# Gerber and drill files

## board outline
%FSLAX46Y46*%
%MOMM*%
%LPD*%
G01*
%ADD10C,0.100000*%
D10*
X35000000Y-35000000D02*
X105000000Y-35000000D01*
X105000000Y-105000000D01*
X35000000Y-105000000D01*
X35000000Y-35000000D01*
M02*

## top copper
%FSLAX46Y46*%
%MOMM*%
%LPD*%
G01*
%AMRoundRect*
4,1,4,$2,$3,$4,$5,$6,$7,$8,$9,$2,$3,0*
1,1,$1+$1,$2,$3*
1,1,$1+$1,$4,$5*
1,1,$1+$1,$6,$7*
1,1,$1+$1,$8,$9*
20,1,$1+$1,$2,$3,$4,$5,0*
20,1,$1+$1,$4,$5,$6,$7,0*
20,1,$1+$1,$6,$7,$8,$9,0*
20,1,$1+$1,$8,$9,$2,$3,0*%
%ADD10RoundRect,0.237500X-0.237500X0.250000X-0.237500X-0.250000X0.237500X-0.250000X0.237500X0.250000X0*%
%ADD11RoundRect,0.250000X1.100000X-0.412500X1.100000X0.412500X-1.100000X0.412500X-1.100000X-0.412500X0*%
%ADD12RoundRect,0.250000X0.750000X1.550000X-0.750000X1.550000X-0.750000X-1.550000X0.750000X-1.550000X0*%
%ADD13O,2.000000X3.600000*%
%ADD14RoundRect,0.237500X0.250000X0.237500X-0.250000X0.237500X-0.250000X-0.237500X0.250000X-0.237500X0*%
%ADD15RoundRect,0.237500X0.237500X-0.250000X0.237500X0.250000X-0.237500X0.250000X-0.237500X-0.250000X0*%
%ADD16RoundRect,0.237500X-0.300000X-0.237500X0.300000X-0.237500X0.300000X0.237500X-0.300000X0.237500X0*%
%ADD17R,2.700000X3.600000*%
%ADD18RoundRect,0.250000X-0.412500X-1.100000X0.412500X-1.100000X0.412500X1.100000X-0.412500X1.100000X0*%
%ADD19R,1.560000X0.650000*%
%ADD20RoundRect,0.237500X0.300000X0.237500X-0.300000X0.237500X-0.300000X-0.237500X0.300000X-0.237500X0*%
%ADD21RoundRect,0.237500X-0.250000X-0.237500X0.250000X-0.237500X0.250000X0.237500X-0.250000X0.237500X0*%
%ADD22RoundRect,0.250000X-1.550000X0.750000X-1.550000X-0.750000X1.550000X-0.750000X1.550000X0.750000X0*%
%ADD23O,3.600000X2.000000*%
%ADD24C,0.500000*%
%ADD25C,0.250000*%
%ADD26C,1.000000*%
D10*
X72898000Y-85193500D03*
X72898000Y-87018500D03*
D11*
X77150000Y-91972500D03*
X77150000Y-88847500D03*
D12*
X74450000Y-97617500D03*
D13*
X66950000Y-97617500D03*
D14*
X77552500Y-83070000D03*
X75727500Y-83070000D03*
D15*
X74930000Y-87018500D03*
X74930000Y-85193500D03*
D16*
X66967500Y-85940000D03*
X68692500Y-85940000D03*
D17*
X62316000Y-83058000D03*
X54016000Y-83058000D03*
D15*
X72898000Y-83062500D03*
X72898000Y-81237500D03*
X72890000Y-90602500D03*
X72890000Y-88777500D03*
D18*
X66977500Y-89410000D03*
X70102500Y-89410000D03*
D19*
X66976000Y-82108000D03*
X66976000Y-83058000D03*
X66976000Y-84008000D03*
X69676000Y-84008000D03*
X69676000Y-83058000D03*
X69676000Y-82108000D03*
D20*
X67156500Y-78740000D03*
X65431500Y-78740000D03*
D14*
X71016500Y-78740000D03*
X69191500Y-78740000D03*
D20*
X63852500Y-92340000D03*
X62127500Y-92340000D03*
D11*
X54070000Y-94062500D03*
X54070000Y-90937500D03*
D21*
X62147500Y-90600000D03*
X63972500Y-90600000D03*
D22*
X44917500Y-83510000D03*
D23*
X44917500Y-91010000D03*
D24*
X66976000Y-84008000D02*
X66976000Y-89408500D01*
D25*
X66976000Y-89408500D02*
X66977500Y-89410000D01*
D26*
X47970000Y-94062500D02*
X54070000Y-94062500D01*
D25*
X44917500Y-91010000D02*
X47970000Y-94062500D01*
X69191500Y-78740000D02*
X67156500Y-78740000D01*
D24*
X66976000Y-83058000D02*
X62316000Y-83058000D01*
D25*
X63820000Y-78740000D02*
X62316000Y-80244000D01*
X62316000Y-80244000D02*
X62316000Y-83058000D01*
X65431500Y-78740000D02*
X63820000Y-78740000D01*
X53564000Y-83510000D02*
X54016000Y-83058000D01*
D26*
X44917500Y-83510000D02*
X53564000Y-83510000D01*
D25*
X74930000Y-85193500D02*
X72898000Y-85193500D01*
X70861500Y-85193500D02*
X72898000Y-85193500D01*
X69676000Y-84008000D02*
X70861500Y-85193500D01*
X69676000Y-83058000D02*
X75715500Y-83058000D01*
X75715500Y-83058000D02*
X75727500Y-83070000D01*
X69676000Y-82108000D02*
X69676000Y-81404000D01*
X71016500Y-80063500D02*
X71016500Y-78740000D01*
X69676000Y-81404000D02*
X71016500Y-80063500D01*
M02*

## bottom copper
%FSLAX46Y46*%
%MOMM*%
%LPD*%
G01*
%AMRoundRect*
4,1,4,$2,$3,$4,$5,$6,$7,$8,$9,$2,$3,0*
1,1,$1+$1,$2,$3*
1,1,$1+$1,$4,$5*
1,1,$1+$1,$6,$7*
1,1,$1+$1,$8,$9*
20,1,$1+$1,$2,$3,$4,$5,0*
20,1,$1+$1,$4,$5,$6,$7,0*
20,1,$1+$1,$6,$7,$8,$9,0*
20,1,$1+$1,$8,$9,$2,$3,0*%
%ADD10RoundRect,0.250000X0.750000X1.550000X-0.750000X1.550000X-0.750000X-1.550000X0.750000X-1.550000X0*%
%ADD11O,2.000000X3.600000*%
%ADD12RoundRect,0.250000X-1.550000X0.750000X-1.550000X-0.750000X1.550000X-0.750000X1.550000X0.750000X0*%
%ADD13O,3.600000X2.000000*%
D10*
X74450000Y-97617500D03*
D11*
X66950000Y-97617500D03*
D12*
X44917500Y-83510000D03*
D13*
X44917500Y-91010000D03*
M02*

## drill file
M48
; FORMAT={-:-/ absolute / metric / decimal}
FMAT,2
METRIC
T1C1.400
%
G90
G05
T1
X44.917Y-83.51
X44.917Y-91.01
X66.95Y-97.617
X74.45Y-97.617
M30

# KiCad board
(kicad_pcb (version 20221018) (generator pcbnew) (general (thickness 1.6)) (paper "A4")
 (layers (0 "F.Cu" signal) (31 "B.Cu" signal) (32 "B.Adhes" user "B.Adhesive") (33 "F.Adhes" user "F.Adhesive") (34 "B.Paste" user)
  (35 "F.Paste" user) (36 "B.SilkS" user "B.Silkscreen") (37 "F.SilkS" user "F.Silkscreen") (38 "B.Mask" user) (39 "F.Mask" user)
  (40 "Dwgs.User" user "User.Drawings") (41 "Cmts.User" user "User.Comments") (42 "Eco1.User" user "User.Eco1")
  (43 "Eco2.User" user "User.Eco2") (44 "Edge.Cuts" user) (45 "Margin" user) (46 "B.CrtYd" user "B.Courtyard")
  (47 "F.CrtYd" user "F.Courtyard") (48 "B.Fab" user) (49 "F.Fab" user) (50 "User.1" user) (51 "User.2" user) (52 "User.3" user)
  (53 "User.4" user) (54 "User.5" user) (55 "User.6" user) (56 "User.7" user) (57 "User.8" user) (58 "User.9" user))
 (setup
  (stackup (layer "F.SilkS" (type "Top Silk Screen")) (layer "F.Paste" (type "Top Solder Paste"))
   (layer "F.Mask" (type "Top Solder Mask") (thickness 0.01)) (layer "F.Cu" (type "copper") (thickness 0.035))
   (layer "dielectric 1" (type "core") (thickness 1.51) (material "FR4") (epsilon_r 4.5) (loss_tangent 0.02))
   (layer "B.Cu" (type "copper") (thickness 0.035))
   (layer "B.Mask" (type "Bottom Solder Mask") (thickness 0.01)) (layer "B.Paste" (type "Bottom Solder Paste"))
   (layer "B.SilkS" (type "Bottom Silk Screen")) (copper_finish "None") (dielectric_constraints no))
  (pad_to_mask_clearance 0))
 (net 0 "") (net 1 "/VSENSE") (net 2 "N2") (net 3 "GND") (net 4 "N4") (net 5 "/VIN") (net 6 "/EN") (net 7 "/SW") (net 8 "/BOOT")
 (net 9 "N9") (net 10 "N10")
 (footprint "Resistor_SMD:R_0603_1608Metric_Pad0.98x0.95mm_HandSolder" (layer "F.Cu") (at 72.898 86.106 -90)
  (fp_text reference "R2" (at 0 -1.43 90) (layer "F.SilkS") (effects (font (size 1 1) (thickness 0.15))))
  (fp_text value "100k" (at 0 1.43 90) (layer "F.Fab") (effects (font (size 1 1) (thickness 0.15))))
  (pad "1" smd roundrect (at -0.9125 0 270) (size 0.975 0.95) (layers "F.Cu" "F.Paste" "F.Mask") (roundrect_rratio 0.25) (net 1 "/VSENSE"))
  (pad "2" smd roundrect (at 0.9125 0 270) (size 0.975 0.95) (layers "F.Cu" "F.Paste" "F.Mask") (roundrect_rratio 0.25) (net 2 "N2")))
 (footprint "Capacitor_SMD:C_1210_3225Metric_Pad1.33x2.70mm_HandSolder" (layer "F.Cu") (at 77.15 90.41 90)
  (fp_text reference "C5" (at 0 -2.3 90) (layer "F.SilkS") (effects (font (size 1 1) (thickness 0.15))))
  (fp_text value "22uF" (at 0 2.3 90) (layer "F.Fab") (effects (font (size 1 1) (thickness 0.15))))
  (pad "1" smd roundrect (at -1.5625 0 90) (size 1.325 2.7) (layers "F.Cu" "F.Paste" "F.Mask") (roundrect_rratio 0.188679) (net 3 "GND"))
  (pad "2" smd roundrect (at 1.5625 0 90) (size 1.325 2.7) (layers "F.Cu" "F.Paste" "F.Mask") (roundrect_rratio 0.188679) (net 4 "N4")))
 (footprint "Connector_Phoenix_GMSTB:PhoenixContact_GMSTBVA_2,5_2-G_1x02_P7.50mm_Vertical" (layer "F.Cu") (at 70.76 97.6175 180)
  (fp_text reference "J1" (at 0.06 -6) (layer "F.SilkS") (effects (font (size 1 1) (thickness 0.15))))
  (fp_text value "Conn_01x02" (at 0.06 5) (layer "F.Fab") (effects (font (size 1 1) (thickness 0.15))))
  (pad "1" thru_hole roundrect (at -3.69 0 180) (size 2 3.6) (drill 1.4) (layers "*.Cu" "*.Mask") (roundrect_rratio 0.125) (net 3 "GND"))
  (pad "2" thru_hole oval (at 3.81 0 180) (size 2 3.6) (drill 1.4) (layers "*.Cu" "*.Mask") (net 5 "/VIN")))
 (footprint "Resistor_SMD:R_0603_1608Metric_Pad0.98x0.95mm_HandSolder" (layer "F.Cu") (at 76.64 83.07 180)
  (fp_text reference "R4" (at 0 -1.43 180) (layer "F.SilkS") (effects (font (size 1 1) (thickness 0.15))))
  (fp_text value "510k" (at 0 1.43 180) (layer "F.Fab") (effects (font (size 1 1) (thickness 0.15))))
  (pad "1" smd roundrect (at -0.9125 0 180) (size 0.975 0.95) (layers "F.Cu" "F.Paste" "F.Mask") (roundrect_rratio 0.25) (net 5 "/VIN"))
  (pad "2" smd roundrect (at 0.9125 0 180) (size 0.975 0.95) (layers "F.Cu" "F.Paste" "F.Mask") (roundrect_rratio 0.25) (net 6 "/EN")))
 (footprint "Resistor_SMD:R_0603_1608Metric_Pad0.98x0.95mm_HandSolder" (layer "F.Cu") (at 74.93 86.106 90)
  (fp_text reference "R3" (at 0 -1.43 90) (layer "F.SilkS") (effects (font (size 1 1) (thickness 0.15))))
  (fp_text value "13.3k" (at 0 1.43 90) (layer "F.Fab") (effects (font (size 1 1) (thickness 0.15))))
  (pad "1" smd roundrect (at -0.9125 0 90) (size 0.975 0.95) (layers "F.Cu" "F.Paste" "F.Mask") (roundrect_rratio 0.25) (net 3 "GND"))
  (pad "2" smd roundrect (at 0.9125 0 90) (size 0.975 0.95) (layers "F.Cu" "F.Paste" "F.Mask") (roundrect_rratio 0.25) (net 1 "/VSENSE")))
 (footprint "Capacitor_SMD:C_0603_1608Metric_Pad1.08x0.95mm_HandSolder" (layer "F.Cu") (at 67.83 85.94)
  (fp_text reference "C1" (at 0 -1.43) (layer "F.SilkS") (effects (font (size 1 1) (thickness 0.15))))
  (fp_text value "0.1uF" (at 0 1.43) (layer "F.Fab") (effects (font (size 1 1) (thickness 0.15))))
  (pad "1" smd roundrect (at -0.8625 0) (size 1.075 0.95) (layers "F.Cu" "F.Paste" "F.Mask") (roundrect_rratio 0.25) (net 5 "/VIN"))
  (pad "2" smd roundrect (at 0.8625 0) (size 1.075 0.95) (layers "F.Cu" "F.Paste" "F.Mask") (roundrect_rratio 0.25) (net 3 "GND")))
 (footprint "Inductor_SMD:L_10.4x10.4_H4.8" (layer "F.Cu") (at 58.166 83.058 180)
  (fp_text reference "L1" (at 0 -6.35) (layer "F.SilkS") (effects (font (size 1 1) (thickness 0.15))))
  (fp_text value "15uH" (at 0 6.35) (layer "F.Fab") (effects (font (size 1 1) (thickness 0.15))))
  (pad "1" smd rect (at -4.15 0 180) (size 2.7 3.6) (layers "F.Cu" "F.Paste" "F.Mask") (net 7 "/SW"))
  (pad "2" smd rect (at 4.15 0 180) (size 2.7 3.6) (layers "F.Cu" "F.Paste" "F.Mask") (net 4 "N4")))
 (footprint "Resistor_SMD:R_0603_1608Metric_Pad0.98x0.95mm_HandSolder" (layer "F.Cu") (at 72.898 82.15 90)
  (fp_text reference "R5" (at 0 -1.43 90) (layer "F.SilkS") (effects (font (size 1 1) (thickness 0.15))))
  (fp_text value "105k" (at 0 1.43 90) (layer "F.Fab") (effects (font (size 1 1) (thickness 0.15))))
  (pad "1" smd roundrect (at -0.9125 0 90) (size 0.975 0.95) (layers "F.Cu" "F.Paste" "F.Mask") (roundrect_rratio 0.25) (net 6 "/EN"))
  (pad "2" smd roundrect (at 0.9125 0 90) (size 0.975 0.95) (layers "F.Cu" "F.Paste" "F.Mask") (roundrect_rratio 0.25) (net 3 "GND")))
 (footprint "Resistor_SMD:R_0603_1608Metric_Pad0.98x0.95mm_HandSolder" (layer "F.Cu") (at 72.89 89.69 90)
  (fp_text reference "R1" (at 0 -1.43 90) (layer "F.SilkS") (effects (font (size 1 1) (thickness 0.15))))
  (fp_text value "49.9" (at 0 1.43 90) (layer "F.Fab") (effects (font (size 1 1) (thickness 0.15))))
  (pad "1" smd roundrect (at -0.9125 0 90) (size 0.975 0.95) (layers "F.Cu" "F.Paste" "F.Mask") (roundrect_rratio 0.25) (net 2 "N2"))
  (pad "2" smd roundrect (at 0.9125 0 90) (size 0.975 0.95) (layers "F.Cu" "F.Paste" "F.Mask") (roundrect_rratio 0.25) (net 4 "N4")))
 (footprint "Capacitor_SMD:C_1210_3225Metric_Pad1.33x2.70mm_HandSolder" (layer "F.Cu") (at 68.54 89.41)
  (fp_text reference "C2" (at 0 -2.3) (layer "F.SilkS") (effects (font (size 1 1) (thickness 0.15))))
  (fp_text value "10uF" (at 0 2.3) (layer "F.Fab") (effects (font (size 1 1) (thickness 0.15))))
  (pad "1" smd roundrect (at -1.5625 0) (size 1.325 2.7) (layers "F.Cu" "F.Paste" "F.Mask") (roundrect_rratio 0.188679) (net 5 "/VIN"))
  (pad "2" smd roundrect (at 1.5625 0) (size 1.325 2.7) (layers "F.Cu" "F.Paste" "F.Mask") (roundrect_rratio 0.188679) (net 3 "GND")))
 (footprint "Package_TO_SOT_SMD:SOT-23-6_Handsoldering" (layer "F.Cu") (at 68.326 83.058)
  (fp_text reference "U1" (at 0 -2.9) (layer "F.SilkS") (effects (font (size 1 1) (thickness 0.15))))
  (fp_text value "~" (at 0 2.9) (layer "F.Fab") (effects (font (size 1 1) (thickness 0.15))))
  (pad "1" smd rect (at -1.35 -0.95) (size 1.56 0.65) (layers "F.Cu" "F.Paste" "F.Mask") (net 3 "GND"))
  (pad "2" smd rect (at -1.35 0) (size 1.56 0.65) (layers "F.Cu" "F.Paste" "F.Mask") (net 7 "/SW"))
  (pad "3" smd rect (at -1.35 0.95) (size 1.56 0.65) (layers "F.Cu" "F.Paste" "F.Mask") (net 5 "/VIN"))
  (pad "4" smd rect (at 1.35 0.95) (size 1.56 0.65) (layers "F.Cu" "F.Paste" "F.Mask") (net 1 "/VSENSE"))
  (pad "5" smd rect (at 1.35 0) (size 1.56 0.65) (layers "F.Cu" "F.Paste" "F.Mask") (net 6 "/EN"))
  (pad "6" smd rect (at 1.35 -0.95) (size 1.56 0.65) (layers "F.Cu" "F.Paste" "F.Mask") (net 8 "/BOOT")))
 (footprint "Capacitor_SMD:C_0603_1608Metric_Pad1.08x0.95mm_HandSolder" (layer "F.Cu") (at 66.294 78.74 180)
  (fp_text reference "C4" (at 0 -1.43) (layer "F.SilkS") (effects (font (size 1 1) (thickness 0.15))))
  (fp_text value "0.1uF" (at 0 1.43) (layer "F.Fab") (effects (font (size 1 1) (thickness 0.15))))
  (pad "1" smd roundrect (at -0.8625 0 180) (size 1.075 0.95) (layers "F.Cu" "F.Paste" "F.Mask") (roundrect_rratio 0.25) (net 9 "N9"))
  (pad "2" smd roundrect (at 0.8625 0 180) (size 1.075 0.95) (layers "F.Cu" "F.Paste" "F.Mask") (roundrect_rratio 0.25) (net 7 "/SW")))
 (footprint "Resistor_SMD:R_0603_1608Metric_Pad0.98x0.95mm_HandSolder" (layer "F.Cu") (at 70.104 78.74 180)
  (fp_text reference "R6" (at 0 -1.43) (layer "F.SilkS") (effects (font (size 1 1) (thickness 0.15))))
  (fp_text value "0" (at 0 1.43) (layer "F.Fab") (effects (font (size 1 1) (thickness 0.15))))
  (pad "1" smd roundrect (at -0.9125 0 180) (size 0.975 0.95) (layers "F.Cu" "F.Paste" "F.Mask") (roundrect_rratio 0.25) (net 8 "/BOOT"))
  (pad "2" smd roundrect (at 0.9125 0 180) (size 0.975 0.95) (layers "F.Cu" "F.Paste" "F.Mask") (roundrect_rratio 0.25) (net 9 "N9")))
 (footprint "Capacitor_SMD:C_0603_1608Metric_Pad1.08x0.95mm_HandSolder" (layer "F.Cu") (at 62.99 92.34 180)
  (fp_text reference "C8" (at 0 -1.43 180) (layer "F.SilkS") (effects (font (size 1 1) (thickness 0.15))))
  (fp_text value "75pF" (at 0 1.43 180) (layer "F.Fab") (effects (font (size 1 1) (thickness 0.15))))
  (pad "1" smd roundrect (at -0.8625 0 180) (size 1.075 0.95) (layers "F.Cu" "F.Paste" "F.Mask") (roundrect_rratio 0.25) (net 1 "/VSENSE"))
  (pad "2" smd roundrect (at 0.8625 0 180) (size 1.075 0.95) (layers "F.Cu" "F.Paste" "F.Mask") (roundrect_rratio 0.25) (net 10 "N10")))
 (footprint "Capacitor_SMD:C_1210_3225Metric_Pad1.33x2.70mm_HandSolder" (layer "F.Cu") (at 54.07 92.5 90)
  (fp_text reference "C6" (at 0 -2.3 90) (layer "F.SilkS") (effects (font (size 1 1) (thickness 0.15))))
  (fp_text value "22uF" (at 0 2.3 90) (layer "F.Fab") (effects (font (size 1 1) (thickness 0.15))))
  (pad "1" smd roundrect (at -1.5625 0 90) (size 1.325 2.7) (layers "F.Cu" "F.Paste" "F.Mask") (roundrect_rratio 0.188679) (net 3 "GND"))
  (pad "2" smd roundrect (at 1.5625 0 90) (size 1.325 2.7) (layers "F.Cu" "F.Paste" "F.Mask") (roundrect_rratio 0.188679) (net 4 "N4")))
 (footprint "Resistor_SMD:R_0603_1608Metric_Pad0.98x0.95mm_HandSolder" (layer "F.Cu") (at 63.06 90.6)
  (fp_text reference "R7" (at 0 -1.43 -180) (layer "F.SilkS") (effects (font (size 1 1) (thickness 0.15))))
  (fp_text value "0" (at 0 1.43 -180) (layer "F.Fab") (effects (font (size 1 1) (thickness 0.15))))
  (pad "1" smd roundrect (at -0.9125 0) (size 0.975 0.95) (layers "F.Cu" "F.Paste" "F.Mask") (roundrect_rratio 0.25) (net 10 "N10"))
  (pad "2" smd roundrect (at 0.9125 0) (size 0.975 0.95) (layers "F.Cu" "F.Paste" "F.Mask") (roundrect_rratio 0.25) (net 2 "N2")))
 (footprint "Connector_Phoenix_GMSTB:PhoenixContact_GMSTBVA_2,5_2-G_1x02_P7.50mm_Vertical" (layer "F.Cu") (at 44.9175 87.2 -90)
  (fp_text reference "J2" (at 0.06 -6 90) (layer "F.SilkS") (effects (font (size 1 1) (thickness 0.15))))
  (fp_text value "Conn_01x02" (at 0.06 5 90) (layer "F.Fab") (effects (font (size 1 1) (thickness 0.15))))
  (pad "1" thru_hole roundrect (at -3.69 0 270) (size 2 3.6) (drill 1.4) (layers "*.Cu" "*.Mask") (roundrect_rratio 0.125) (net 4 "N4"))
  (pad "2" thru_hole oval (at 3.81 0 270) (size 2 3.6) (drill 1.4) (layers "*.Cu" "*.Mask") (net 3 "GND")))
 (gr_rect (start 35 35) (end 105 105) (stroke (width 0.1) (type default)) (fill none) (layer "Edge.Cuts"))
 (segment (start 66.976 84.008) (end 66.976 89.4085) (width 0.5) (layer "F.Cu") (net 5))
 (segment (start 66.976 89.4085) (end 66.9775 89.41) (width 0.25) (layer "F.Cu") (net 5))
 (segment (start 47.97 94.0625) (end 54.07 94.0625) (width 1) (layer "F.Cu") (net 3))
 (segment (start 44.9175 91.01) (end 47.97 94.0625) (width 0.25) (layer "F.Cu") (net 3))
 (segment (start 69.1915 78.74) (end 67.1565 78.74) (width 0.25) (layer "F.Cu") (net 9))
 (segment (start 66.976 83.058) (end 62.316 83.058) (width 0.5) (layer "F.Cu") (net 7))
 (segment (start 63.82 78.74) (end 62.316 80.244) (width 0.25) (layer "F.Cu") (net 7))
 (segment (start 62.316 80.244) (end 62.316 83.058) (width 0.25) (layer "F.Cu") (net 7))
 (segment (start 65.4315 78.74) (end 63.82 78.74) (width 0.25) (layer "F.Cu") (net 7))
 (segment (start 53.564 83.51) (end 54.016 83.058) (width 0.25) (layer "F.Cu") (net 4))
 (segment (start 44.9175 83.51) (end 53.564 83.51) (width 1) (layer "F.Cu") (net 4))
 (segment (start 74.93 85.1935) (end 72.898 85.1935) (width 0.25) (layer "F.Cu") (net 1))
 (segment (start 70.8615 85.1935) (end 72.898 85.1935) (width 0.25) (layer "F.Cu") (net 1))
 (segment (start 69.676 84.008) (end 70.8615 85.1935) (width 0.25) (layer "F.Cu") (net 1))
 (segment (start 69.676 83.058) (end 75.7155 83.058) (width 0.25) (layer "F.Cu") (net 6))
 (segment (start 75.7155 83.058) (end 75.7275 83.07) (width 0.25) (layer "F.Cu") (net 6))
 (segment (start 69.676 82.108) (end 69.676 81.404) (width 0.25) (layer "F.Cu") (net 8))
 (segment (start 71.0165 80.0635) (end 71.0165 78.74) (width 0.25) (layer "F.Cu") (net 8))
 (segment (start 69.676 81.404) (end 71.0165 80.0635) (width 0.25) (layer "F.Cu") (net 8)))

